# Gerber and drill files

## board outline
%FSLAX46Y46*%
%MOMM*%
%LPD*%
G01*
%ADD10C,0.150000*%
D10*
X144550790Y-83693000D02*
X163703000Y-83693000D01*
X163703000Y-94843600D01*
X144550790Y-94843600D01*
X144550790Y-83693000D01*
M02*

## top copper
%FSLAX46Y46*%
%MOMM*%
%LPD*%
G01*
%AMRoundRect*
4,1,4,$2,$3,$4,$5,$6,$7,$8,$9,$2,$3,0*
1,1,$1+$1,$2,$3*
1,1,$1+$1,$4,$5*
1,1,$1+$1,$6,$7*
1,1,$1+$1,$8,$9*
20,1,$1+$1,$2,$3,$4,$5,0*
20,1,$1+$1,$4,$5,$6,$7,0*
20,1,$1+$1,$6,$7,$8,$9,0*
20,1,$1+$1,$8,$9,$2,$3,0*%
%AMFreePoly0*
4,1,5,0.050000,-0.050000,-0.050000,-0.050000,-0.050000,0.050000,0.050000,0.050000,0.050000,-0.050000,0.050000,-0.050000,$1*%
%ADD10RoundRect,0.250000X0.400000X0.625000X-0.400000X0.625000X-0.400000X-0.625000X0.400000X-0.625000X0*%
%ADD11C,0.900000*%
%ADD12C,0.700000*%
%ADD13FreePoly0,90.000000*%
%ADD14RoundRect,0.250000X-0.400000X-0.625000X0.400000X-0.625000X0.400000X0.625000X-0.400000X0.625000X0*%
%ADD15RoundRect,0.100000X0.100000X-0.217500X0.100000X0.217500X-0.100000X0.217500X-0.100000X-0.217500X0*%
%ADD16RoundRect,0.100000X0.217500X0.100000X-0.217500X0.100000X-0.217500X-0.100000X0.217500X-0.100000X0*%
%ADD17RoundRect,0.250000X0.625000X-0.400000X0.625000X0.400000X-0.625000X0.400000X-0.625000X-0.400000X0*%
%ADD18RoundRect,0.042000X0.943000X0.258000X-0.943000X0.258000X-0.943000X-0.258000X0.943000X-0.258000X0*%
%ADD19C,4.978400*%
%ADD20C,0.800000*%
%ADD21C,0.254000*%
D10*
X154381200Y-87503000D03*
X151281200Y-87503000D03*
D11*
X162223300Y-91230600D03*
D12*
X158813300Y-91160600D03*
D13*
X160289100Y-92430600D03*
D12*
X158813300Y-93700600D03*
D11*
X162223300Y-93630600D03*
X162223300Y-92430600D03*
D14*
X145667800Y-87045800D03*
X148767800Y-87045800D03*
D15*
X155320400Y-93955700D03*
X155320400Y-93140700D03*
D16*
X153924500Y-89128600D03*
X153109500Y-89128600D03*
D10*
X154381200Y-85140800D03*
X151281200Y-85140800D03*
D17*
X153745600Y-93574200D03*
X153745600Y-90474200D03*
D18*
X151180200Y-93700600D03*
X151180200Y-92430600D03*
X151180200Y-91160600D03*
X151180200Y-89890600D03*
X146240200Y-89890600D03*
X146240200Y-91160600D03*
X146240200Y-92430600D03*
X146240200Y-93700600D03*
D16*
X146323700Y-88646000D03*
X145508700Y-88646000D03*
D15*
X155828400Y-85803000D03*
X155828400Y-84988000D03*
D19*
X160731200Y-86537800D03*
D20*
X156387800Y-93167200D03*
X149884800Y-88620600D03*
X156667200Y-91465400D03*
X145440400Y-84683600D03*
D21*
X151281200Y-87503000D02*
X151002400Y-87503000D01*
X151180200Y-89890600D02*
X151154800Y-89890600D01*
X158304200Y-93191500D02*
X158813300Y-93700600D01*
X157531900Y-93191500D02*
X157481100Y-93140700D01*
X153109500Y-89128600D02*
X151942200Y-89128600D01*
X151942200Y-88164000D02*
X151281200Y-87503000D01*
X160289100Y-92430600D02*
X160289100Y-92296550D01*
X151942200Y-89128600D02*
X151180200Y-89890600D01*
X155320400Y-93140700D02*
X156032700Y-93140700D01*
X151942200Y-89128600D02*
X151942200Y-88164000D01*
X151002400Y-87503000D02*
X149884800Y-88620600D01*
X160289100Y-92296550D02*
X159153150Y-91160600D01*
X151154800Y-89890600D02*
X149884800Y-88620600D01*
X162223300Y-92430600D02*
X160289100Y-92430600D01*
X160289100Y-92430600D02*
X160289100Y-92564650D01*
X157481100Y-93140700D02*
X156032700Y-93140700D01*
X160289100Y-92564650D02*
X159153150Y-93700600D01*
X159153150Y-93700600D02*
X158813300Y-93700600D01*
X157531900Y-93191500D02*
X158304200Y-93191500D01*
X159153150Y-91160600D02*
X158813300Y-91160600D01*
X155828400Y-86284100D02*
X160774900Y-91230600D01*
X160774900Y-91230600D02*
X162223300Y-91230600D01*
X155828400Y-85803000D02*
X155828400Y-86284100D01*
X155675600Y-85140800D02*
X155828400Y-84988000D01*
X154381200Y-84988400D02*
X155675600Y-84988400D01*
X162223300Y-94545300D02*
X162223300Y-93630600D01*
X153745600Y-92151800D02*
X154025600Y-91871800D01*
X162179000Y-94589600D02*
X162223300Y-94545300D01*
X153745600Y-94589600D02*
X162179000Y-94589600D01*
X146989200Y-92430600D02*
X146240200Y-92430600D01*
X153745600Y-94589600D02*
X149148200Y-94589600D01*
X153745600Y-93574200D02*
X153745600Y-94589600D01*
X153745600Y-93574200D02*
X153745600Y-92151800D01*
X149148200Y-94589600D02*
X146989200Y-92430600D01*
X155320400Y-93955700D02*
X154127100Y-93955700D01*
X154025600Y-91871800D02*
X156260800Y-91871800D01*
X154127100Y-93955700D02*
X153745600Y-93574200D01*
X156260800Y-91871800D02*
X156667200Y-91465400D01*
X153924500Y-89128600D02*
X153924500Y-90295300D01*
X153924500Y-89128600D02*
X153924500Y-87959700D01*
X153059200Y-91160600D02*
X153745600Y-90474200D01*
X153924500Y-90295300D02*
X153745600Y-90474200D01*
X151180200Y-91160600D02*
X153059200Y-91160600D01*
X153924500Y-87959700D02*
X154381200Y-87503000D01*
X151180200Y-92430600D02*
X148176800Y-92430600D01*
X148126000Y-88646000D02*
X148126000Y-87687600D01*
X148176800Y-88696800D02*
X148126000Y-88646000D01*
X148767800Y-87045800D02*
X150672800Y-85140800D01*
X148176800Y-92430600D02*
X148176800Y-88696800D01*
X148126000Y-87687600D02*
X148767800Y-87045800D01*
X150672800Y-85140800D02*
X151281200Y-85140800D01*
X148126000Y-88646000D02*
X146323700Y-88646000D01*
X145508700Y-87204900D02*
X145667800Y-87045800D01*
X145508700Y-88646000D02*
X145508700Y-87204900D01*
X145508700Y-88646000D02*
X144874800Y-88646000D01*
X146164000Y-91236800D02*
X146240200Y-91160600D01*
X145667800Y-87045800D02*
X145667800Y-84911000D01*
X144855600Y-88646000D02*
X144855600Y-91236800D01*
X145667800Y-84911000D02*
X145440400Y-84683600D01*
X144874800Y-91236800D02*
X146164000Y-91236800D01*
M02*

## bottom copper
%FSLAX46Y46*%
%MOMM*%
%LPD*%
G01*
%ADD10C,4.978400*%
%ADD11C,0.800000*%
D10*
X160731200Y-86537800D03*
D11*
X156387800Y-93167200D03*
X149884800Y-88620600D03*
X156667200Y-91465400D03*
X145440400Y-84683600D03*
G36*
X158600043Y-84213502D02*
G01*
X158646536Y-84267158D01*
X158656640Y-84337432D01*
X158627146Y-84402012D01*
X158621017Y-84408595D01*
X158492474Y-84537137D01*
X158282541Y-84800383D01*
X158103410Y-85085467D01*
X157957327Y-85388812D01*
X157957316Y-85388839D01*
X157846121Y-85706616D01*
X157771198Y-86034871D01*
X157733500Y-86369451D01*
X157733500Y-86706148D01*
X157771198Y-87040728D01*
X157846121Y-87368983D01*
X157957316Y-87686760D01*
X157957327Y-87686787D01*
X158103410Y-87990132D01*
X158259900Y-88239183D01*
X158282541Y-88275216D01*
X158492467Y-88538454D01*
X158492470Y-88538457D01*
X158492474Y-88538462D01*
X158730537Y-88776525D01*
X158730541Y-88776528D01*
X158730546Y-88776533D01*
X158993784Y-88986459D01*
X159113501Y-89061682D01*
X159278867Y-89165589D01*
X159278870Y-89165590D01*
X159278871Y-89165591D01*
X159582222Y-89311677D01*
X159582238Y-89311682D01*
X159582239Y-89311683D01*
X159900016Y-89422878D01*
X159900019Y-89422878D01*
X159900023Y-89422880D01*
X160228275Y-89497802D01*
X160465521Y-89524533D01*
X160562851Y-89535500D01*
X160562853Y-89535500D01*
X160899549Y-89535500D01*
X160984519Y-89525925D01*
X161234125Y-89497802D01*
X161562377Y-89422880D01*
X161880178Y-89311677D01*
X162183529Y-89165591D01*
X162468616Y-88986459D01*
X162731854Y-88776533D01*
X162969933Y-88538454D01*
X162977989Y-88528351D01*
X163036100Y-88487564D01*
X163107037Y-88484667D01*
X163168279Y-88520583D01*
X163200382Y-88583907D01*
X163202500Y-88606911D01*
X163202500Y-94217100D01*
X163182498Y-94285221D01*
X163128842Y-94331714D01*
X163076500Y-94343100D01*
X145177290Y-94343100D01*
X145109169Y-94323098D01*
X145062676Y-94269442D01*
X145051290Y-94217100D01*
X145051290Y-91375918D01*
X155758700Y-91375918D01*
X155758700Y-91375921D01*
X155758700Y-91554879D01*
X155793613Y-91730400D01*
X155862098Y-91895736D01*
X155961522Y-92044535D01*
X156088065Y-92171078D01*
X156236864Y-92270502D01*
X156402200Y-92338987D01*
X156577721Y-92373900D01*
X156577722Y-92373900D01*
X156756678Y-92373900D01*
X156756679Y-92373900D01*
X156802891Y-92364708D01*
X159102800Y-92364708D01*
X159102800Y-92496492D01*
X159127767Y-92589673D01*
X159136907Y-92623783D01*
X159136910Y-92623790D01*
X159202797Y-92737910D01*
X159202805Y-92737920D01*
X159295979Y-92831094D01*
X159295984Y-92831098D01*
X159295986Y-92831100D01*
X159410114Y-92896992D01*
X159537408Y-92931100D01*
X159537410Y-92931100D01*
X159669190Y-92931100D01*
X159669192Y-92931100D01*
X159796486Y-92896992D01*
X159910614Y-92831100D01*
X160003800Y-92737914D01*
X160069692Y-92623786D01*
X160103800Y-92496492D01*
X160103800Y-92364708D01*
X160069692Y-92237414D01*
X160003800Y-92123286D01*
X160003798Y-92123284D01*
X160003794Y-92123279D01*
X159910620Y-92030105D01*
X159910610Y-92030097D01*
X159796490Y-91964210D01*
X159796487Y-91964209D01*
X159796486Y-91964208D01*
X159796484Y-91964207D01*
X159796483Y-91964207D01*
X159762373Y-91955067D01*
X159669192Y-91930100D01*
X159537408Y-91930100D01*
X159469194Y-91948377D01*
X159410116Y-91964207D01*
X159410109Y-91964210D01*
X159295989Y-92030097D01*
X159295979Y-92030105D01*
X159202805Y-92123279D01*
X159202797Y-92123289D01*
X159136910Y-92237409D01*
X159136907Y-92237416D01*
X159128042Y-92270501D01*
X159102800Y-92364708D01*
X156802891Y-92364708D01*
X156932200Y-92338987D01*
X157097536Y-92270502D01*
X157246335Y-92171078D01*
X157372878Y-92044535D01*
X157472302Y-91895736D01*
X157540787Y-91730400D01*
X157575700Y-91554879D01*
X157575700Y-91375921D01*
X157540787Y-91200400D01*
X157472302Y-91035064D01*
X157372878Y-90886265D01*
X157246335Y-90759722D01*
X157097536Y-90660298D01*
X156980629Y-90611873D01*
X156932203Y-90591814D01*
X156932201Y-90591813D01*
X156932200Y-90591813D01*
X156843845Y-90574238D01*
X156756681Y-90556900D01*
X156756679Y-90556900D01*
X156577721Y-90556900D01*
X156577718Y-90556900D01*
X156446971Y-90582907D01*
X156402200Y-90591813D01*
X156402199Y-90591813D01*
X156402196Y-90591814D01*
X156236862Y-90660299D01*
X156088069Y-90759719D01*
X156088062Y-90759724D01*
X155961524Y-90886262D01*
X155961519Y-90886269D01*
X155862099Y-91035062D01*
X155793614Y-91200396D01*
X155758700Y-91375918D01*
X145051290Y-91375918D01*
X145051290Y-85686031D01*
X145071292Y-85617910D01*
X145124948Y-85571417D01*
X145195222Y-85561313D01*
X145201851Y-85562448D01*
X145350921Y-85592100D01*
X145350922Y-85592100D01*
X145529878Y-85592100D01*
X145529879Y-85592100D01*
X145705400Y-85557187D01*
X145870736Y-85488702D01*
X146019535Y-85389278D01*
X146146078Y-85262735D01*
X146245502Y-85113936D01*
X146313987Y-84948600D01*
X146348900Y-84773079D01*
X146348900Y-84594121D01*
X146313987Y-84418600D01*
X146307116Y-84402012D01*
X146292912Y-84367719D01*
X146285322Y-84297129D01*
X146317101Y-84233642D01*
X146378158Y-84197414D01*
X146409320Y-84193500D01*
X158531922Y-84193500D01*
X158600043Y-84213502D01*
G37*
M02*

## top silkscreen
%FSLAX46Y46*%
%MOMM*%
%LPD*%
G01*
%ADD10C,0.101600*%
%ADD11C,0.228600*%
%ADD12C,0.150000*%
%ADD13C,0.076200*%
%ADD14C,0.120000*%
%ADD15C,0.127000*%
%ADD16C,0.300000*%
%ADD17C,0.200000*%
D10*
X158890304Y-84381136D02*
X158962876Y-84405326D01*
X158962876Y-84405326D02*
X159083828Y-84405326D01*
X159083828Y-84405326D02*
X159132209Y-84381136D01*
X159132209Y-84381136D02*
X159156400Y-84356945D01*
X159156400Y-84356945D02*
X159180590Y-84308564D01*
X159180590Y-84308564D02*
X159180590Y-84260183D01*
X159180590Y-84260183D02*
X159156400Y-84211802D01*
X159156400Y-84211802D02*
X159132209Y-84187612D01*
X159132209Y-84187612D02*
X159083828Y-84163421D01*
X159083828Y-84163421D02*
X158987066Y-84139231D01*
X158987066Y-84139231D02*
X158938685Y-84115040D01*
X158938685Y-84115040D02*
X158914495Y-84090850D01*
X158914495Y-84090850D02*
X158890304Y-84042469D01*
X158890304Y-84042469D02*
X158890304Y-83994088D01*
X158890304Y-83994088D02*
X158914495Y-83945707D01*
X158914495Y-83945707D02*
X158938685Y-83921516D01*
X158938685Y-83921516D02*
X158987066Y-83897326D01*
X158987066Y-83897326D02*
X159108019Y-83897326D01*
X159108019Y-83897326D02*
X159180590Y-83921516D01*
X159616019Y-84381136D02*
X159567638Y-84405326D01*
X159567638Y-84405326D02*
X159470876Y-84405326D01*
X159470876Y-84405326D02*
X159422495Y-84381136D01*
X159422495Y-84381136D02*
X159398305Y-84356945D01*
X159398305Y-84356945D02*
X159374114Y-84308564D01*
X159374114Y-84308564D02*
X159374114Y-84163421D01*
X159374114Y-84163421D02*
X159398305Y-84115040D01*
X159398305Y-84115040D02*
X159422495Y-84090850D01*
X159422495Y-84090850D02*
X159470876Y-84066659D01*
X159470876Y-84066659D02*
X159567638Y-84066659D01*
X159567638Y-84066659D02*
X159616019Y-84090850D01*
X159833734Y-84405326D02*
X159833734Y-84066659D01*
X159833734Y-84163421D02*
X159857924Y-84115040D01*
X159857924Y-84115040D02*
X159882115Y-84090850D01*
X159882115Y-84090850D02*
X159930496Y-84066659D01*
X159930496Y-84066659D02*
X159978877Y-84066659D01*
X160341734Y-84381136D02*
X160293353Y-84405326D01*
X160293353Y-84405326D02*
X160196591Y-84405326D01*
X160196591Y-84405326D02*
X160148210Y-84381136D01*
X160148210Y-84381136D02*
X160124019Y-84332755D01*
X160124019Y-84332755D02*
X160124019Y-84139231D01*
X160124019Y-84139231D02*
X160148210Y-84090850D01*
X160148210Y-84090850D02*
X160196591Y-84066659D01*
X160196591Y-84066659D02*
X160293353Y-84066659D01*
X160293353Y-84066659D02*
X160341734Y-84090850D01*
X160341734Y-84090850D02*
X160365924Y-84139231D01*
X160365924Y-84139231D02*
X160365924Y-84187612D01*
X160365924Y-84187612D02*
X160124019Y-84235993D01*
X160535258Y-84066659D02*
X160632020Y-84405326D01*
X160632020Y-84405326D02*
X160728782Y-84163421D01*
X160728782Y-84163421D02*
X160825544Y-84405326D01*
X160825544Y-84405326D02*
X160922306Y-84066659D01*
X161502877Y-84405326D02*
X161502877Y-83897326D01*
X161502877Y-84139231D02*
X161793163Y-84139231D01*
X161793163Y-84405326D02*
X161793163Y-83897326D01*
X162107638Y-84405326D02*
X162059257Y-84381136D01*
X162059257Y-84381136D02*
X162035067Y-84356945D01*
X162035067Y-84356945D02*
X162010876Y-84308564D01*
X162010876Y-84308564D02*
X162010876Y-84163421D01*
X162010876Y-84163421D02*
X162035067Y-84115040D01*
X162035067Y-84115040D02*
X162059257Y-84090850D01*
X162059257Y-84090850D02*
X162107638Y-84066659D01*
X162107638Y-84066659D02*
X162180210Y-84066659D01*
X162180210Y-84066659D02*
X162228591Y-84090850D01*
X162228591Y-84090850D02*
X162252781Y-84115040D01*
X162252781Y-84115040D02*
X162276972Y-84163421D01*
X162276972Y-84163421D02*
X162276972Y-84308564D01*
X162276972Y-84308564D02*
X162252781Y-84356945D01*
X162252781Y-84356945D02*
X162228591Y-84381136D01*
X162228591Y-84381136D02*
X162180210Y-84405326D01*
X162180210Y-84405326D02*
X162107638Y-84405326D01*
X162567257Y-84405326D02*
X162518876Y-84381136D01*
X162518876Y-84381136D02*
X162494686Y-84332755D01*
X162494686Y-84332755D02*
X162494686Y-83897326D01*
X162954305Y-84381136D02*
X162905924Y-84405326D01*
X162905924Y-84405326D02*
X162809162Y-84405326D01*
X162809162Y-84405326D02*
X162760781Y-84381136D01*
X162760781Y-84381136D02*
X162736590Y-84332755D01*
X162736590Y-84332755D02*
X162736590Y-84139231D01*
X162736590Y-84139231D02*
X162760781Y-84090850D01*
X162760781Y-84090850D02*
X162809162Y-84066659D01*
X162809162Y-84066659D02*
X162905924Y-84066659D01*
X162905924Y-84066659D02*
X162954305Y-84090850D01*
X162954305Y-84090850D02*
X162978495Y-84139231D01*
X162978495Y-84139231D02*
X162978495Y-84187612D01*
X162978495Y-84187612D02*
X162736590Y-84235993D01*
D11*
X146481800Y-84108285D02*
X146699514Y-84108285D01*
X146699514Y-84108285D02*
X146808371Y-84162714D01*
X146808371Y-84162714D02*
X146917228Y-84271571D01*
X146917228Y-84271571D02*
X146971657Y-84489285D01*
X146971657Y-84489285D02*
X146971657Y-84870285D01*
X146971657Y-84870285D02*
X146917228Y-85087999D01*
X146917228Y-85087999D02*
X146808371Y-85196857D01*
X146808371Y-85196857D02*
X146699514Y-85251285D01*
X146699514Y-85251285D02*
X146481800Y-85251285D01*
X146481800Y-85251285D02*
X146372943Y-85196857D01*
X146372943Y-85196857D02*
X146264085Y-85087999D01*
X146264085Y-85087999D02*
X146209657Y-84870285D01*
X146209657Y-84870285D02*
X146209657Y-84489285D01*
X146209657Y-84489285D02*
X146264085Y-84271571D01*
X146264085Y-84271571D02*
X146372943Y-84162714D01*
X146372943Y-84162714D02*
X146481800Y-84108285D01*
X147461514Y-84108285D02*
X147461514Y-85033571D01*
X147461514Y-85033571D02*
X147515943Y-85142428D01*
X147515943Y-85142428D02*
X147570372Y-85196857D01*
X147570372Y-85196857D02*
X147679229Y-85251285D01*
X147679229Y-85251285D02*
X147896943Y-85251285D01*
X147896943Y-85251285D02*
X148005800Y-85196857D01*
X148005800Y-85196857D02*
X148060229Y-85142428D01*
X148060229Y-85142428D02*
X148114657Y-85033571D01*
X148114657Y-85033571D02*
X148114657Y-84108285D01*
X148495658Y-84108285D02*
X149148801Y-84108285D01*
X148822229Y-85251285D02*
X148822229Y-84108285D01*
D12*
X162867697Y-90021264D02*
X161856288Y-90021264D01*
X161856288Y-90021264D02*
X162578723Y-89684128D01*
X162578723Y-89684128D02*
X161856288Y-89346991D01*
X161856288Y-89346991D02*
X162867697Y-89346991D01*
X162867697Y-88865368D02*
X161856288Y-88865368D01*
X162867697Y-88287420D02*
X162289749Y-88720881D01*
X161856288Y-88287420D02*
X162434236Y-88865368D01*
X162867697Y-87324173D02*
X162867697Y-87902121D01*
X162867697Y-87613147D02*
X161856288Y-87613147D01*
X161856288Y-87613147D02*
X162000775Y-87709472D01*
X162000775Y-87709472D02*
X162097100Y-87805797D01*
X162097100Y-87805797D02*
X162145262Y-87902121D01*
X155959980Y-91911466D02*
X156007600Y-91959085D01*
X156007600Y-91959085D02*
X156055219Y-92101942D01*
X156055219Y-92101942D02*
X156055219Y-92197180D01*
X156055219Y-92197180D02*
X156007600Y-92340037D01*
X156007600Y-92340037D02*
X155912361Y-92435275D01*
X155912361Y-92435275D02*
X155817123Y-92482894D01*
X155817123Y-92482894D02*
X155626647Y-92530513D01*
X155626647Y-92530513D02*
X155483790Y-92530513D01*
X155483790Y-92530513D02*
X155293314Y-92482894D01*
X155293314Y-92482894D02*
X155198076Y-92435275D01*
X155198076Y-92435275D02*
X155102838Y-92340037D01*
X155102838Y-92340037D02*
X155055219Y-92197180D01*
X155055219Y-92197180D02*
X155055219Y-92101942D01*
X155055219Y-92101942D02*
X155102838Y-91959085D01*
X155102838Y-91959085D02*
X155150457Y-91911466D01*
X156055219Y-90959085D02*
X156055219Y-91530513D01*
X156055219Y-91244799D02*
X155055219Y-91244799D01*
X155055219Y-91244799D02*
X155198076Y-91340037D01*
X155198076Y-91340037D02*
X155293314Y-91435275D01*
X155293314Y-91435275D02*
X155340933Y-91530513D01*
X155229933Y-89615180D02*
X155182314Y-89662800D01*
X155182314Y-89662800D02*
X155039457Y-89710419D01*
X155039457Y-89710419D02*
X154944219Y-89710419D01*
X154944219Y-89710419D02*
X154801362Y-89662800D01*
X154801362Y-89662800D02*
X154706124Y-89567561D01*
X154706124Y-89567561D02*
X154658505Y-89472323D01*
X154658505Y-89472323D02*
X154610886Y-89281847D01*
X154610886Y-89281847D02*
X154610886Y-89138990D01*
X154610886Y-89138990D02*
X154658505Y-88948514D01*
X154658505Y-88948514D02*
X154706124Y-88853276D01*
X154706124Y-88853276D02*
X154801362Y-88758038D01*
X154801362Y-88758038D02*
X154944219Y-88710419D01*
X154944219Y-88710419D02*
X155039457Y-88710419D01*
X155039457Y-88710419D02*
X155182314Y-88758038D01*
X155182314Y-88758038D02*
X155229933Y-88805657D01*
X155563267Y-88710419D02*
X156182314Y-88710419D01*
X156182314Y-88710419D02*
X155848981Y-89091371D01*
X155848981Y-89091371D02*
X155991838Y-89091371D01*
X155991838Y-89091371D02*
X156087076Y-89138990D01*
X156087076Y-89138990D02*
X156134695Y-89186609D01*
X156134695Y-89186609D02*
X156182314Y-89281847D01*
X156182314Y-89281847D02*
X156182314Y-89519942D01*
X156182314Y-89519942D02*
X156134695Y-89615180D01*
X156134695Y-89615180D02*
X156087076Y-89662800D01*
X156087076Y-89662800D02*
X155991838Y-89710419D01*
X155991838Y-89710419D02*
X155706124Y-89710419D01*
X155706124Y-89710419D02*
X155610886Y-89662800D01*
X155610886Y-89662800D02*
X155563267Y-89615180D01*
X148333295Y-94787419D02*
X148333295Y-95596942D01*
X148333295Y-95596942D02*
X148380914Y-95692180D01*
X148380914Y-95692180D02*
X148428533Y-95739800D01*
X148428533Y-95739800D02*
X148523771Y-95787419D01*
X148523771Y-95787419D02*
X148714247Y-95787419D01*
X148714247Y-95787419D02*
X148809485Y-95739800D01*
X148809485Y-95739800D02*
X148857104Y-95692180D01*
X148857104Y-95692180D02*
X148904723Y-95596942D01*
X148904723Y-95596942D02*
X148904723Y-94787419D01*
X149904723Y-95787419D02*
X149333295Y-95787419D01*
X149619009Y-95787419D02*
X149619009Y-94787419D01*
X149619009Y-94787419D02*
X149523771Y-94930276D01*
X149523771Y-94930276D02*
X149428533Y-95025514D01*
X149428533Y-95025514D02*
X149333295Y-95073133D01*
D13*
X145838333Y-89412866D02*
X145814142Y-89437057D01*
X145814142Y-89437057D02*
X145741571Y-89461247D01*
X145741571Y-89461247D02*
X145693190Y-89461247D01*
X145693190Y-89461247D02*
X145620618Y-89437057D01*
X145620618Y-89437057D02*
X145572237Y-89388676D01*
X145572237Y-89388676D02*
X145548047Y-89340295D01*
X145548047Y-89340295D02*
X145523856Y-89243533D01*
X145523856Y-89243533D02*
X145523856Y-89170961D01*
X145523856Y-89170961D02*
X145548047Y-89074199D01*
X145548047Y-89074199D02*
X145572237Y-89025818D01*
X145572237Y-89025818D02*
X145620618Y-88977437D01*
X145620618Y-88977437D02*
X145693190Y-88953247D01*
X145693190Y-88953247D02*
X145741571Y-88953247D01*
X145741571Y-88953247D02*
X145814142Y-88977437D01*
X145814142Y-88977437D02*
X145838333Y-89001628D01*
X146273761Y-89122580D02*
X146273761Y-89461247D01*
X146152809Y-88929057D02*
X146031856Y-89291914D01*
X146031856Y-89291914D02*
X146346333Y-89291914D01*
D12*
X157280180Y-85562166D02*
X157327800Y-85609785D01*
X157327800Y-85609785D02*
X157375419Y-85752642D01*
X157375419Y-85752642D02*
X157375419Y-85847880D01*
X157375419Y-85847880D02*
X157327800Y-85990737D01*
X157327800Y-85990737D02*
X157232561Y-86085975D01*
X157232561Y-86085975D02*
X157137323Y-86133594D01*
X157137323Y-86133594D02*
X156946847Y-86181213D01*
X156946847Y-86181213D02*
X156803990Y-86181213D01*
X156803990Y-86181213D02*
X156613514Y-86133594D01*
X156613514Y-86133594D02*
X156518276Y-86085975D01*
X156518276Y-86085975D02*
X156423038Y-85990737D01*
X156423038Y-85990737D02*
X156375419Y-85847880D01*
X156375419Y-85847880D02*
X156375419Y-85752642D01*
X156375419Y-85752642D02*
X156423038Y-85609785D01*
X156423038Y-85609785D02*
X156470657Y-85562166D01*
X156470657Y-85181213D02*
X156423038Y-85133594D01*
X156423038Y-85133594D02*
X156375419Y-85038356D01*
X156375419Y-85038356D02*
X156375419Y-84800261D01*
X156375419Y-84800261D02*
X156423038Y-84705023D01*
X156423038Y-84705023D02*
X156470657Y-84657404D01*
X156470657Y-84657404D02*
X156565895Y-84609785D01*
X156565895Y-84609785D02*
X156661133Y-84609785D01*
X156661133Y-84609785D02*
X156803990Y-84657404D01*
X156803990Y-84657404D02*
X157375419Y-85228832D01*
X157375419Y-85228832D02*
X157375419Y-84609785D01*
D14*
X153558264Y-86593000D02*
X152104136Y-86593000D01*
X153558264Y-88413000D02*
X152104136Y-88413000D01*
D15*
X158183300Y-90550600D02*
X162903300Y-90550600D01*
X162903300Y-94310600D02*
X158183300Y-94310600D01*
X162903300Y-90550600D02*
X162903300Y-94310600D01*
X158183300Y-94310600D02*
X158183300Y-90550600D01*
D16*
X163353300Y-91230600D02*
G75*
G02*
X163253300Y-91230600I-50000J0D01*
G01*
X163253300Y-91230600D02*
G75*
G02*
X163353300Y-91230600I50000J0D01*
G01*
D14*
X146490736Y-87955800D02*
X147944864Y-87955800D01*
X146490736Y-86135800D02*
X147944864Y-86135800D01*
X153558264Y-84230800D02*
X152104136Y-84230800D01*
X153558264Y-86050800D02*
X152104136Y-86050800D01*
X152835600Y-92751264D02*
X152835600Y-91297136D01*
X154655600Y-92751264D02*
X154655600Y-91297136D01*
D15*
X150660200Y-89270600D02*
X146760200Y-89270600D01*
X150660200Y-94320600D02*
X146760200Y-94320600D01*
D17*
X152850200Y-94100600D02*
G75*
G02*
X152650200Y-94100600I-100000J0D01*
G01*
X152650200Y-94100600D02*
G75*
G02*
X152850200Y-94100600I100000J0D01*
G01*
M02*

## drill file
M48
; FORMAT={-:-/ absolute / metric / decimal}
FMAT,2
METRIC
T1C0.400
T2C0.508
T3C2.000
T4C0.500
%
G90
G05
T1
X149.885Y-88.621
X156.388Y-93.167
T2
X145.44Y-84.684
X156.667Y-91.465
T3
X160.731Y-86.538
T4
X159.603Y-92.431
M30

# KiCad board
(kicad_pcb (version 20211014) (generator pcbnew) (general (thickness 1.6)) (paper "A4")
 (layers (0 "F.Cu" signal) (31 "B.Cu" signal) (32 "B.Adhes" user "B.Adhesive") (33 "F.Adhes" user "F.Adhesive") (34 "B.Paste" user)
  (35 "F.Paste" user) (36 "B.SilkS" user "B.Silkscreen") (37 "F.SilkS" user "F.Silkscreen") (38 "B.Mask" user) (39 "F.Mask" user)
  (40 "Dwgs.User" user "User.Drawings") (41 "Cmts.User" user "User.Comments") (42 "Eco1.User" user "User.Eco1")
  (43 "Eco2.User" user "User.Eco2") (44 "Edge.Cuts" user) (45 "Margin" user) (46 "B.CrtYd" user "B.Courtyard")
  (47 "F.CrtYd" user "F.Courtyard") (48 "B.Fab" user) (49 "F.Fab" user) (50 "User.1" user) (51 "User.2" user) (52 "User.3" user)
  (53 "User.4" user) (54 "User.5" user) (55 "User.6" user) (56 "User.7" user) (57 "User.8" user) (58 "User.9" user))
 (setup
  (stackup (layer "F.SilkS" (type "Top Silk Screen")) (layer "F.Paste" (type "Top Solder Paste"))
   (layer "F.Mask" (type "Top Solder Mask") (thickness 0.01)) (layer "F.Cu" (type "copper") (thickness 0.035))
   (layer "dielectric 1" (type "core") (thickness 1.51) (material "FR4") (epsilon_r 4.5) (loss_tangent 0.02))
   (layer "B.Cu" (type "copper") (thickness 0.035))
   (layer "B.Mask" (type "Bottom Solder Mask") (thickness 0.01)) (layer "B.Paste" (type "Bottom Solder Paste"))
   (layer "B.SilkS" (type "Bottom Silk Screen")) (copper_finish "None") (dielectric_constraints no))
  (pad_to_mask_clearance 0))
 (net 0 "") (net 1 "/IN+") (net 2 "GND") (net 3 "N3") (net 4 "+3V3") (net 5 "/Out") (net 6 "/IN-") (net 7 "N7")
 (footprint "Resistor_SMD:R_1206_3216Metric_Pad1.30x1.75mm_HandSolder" (layer "F.Cu") (at 152.8312 87.503 180)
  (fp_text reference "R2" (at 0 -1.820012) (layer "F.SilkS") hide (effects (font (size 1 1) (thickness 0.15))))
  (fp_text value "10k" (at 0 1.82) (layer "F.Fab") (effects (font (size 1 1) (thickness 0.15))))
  (fp_line (start -0.727064 0.91) (end 0.727064 0.91) (layer "F.SilkS") (width 0.12))
  (fp_line (start -0.727064 -0.91) (end 0.727064 -0.91) (layer "F.SilkS") (width 0.12))
  (pad "1" smd roundrect (at -1.55 0 180) (size 1.3 1.75) (layers "F.Cu" "F.Paste" "F.Mask") (roundrect_rratio 0.1923076923) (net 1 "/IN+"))
  (pad "2" smd roundrect (at 1.55 0 180) (size 1.3 1.75) (layers "F.Cu" "F.Paste" "F.Mask") (roundrect_rratio 0.1923076923) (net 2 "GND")))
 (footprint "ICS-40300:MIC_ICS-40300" (layer "F.Cu") (at 159.6033 92.4306 -90)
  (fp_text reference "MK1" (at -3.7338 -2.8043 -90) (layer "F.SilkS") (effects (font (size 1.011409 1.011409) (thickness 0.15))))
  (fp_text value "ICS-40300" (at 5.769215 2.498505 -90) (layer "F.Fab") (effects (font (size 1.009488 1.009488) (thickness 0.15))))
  (fp_line (start -1.88 1.42) (end -1.88 -3.3) (layer "F.SilkS") (width 0.127))
  (fp_line (start 1.88 -3.3) (end 1.88 1.42) (layer "F.SilkS") (width 0.127))
  (fp_line (start -1.88 -3.3) (end 1.88 -3.3) (layer "F.SilkS") (width 0.127))
  (fp_line (start 1.88 1.42) (end -1.88 1.42) (layer "F.SilkS") (width 0.127))
  (fp_circle (center -1.2 -3.7) (end -1.15 -3.7) (layer "F.SilkS") (width 0.3) (fill none))
  (pad "" np_thru_hole circle (at 0 0 270) (size 0.5 0.5) (drill 0.5) (layers *.Cu *.Mask))
  (pad "1" smd circle (at -1.2 -2.62 180) (size 0.9 0.9) (layers "F.Cu" "F.Mask") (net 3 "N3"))
  (pad "2" smd circle (at -1.27 0.79 180) (size 0.7 0.7) (layers "F.Cu" "F.Mask") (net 2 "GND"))
  (pad "3" smd custom (at 0 -0.6858 90) (size 0.1 0.1) (layers "F.Cu") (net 2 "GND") (zone_connect 0)
   (options (clearance outline) (anchor rect)) (primitives))
  (pad "4" smd circle (at 1.27 0.79 180) (size 0.7 0.7) (layers "F.Cu" "F.Mask") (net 2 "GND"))
  (pad "5" smd circle (at 1.2 -2.62 180) (size 0.9 0.9) (layers "F.Cu" "F.Mask") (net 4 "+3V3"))
  (pad "6" smd circle (at 0 -2.62 180) (size 0.9 0.9) (layers "F.Cu" "F.Mask") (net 2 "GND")))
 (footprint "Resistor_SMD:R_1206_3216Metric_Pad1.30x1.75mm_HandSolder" (layer "F.Cu") (at 147.2178 87.0458)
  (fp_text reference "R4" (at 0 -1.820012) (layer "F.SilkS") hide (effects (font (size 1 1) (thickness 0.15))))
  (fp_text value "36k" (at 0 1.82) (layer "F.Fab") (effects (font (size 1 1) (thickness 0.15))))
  (fp_line (start -0.727064 0.91) (end 0.727064 0.91) (layer "F.SilkS") (width 0.12))
  (fp_line (start -0.727064 -0.91) (end 0.727064 -0.91) (layer "F.SilkS") (width 0.12))
  (pad "1" smd roundrect (at -1.55 0) (size 1.3 1.75) (layers "F.Cu" "F.Paste" "F.Mask") (roundrect_rratio 0.1923076923) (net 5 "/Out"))
  (pad "2" smd roundrect (at 1.55 0) (size 1.3 1.75) (layers "F.Cu" "F.Paste" "F.Mask") (roundrect_rratio 0.1923076923) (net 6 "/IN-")))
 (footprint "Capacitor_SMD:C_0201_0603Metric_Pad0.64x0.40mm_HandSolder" (layer "F.Cu") (at 155.3204 93.5482 90)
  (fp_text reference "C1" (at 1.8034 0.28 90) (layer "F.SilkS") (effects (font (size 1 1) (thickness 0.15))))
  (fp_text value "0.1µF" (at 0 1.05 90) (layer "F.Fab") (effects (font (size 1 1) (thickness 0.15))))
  (pad "" smd roundrect (at 0.4325 0 90) (size 0.458 0.36) (layers "F.Paste") (roundrect_rratio 0.25))
  (pad "" smd roundrect (at -0.4325 0 90) (size 0.458 0.36) (layers "F.Paste") (roundrect_rratio 0.25))
  (pad "1" smd roundrect (at -0.4075 0 90) (size 0.635 0.4) (layers "F.Cu" "F.Mask") (roundrect_rratio 0.25) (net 4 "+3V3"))
  (pad "2" smd roundrect (at 0.4075 0 90) (size 0.635 0.4) (layers "F.Cu" "F.Mask") (roundrect_rratio 0.25) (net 2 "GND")))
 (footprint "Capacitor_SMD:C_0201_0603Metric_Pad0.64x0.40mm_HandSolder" (layer "F.Cu") (at 153.517 89.1286 180)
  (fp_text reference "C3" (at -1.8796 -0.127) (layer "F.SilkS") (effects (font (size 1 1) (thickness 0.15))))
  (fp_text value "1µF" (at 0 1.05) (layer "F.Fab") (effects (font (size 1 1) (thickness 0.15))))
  (pad "" smd roundrect (at -0.4325 0 180) (size 0.458 0.36) (layers "F.Paste") (roundrect_rratio 0.25))
  (pad "" smd roundrect (at 0.4325 0 180) (size 0.458 0.36) (layers "F.Paste") (roundrect_rratio 0.25))
  (pad "1" smd roundrect (at -0.4075 0 180) (size 0.635 0.4) (layers "F.Cu" "F.Mask") (roundrect_rratio 0.25) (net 1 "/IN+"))
  (pad "2" smd roundrect (at 0.4075 0 180) (size 0.635 0.4) (layers "F.Cu" "F.Mask") (roundrect_rratio 0.25) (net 2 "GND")))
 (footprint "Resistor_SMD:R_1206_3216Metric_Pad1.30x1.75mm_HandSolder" (layer "F.Cu") (at 152.8312 85.1408 180)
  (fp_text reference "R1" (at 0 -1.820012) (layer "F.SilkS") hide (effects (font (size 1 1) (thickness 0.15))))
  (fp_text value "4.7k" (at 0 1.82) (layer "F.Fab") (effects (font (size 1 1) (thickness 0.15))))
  (fp_line (start -0.727064 0.91) (end 0.727064 0.91) (layer "F.SilkS") (width 0.12))
  (fp_line (start -0.727064 -0.91) (end 0.727064 -0.91) (layer "F.SilkS") (width 0.12))
  (pad "1" smd roundrect (at -1.55 0 180) (size 1.3 1.75) (layers "F.Cu" "F.Paste" "F.Mask") (roundrect_rratio 0.1923076923) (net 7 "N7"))
  (pad "2" smd roundrect (at 1.55 0 180) (size 1.3 1.75) (layers "F.Cu" "F.Paste" "F.Mask") (roundrect_rratio 0.1923076923) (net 6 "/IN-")))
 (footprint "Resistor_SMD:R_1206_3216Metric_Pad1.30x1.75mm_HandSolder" (layer "F.Cu") (at 153.7456 92.0242 90)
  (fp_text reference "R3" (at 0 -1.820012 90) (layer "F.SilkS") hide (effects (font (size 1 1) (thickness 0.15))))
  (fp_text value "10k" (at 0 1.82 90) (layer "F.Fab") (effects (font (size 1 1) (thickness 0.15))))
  (fp_line (start -0.727064 -0.91) (end 0.727064 -0.91) (layer "F.SilkS") (width 0.12))
  (fp_line (start -0.727064 0.91) (end 0.727064 0.91) (layer "F.SilkS") (width 0.12))
  (pad "1" smd roundrect (at -1.55 0 90) (size 1.3 1.75) (layers "F.Cu" "F.Paste" "F.Mask") (roundrect_rratio 0.1923076923) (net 4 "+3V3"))
  (pad "2" smd roundrect (at 1.55 0 90) (size 1.3 1.75) (layers "F.Cu" "F.Paste" "F.Mask") (roundrect_rratio 0.1923076923) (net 1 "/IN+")))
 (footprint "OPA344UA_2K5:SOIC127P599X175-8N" (layer "F.Cu") (at 148.7102 91.7956 180)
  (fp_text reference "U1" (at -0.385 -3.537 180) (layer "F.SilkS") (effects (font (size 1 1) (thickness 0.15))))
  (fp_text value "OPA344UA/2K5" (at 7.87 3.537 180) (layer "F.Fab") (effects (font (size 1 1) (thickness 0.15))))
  (fp_line (start -1.95 2.525) (end 1.95 2.525) (layer "F.SilkS") (width 0.127))
  (fp_line (start -1.95 -2.525) (end 1.95 -2.525) (layer "F.SilkS") (width 0.127))
  (fp_circle (center -4.04 -2.305) (end -3.94 -2.305) (layer "F.SilkS") (width 0.2) (fill none))
  (pad "1" smd roundrect locked (at -2.47 -1.905 180) (size 1.97 0.6) (layers "F.Cu" "F.Paste" "F.Mask") (roundrect_rratio 0.07))
  (pad "2" smd roundrect locked (at -2.47 -0.635 180) (size 1.97 0.6) (layers "F.Cu" "F.Paste" "F.Mask") (roundrect_rratio 0.07)
   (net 6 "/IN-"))
  (pad "3" smd roundrect locked (at -2.47 0.635 180) (size 1.97 0.6) (layers "F.Cu" "F.Paste" "F.Mask") (roundrect_rratio 0.07)
   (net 1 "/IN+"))
  (pad "4" smd roundrect locked (at -2.47 1.905 180) (size 1.97 0.6) (layers "F.Cu" "F.Paste" "F.Mask") (roundrect_rratio 0.07)
   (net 2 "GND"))
  (pad "5" smd roundrect locked (at 2.47 1.905 180) (size 1.97 0.6) (layers "F.Cu" "F.Paste" "F.Mask") (roundrect_rratio 0.07))
  (pad "6" smd roundrect locked (at 2.47 0.635 180) (size 1.97 0.6) (layers "F.Cu" "F.Paste" "F.Mask") (roundrect_rratio 0.07)
   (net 5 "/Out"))
  (pad "7" smd roundrect locked (at 2.47 -0.635 180) (size 1.97 0.6) (layers "F.Cu" "F.Paste" "F.Mask") (roundrect_rratio 0.07)
   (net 4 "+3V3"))
  (pad "8" smd roundrect locked (at 2.47 -1.905 180) (size 1.97 0.6) (layers "F.Cu" "F.Paste" "F.Mask") (roundrect_rratio 0.07)))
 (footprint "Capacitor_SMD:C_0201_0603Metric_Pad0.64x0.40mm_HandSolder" (layer "F.Cu") (at 145.9162 88.646 180)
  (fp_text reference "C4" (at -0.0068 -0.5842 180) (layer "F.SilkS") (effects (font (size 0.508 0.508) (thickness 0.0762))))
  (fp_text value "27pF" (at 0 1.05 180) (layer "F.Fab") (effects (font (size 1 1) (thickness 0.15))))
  (pad "" smd roundrect (at -0.4325 0 180) (size 0.458 0.36) (layers "F.Paste") (roundrect_rratio 0.25))
  (pad "" smd roundrect (at 0.4325 0 180) (size 0.458 0.36) (layers "F.Paste") (roundrect_rratio 0.25))
  (pad "1" smd roundrect (at -0.4075 0 180) (size 0.635 0.4) (layers "F.Cu" "F.Mask") (roundrect_rratio 0.25) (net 6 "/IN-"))
  (pad "2" smd roundrect (at 0.4075 0 180) (size 0.635 0.4) (layers "F.Cu" "F.Mask") (roundrect_rratio 0.25) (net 5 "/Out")))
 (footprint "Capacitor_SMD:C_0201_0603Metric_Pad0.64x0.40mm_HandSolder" (layer "F.Cu") (at 155.8284 85.3955 90)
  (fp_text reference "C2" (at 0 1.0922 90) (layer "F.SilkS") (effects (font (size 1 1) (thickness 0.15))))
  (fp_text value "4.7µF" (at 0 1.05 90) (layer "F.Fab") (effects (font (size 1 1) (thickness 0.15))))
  (pad "" smd roundrect (at -0.4325 0 90) (size 0.458 0.36) (layers "F.Paste") (roundrect_rratio 0.25))
  (pad "" smd roundrect (at 0.4325 0 90) (size 0.458 0.36) (layers "F.Paste") (roundrect_rratio 0.25))
  (pad "1" smd roundrect (at -0.4075 0 90) (size 0.635 0.4) (layers "F.Cu" "F.Mask") (roundrect_rratio 0.25) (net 3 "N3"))
  (pad "2" smd roundrect (at 0.4075 0 90) (size 0.635 0.4) (layers "F.Cu" "F.Mask") (roundrect_rratio 0.25) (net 7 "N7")))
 (gr_rect (start 144.55079 94.8436) (end 163.703 83.693) (layer "Edge.Cuts") (width 0.15) (fill none))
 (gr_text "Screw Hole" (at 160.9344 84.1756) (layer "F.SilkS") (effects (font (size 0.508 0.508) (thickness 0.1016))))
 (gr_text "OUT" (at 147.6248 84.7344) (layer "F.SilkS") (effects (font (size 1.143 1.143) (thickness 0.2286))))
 (via (at 160.7312 86.5378) (size 4.9784) (drill 2.000001) (layers "F.Cu" "B.Cu") (free) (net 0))
 (segment (start 151.2812 87.503) (end 151.0024 87.503) (width 0.254) (layer "F.Cu") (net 2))
 (segment (start 151.1802 89.8906) (end 151.1548 89.8906) (width 0.254) (layer "F.Cu") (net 2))
 (segment (start 158.3042 93.1915) (end 158.8133 93.7006) (width 0.254) (layer "F.Cu") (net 2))
 (segment (start 157.5319 93.1915) (end 157.4811 93.1407) (width 0.254) (layer "F.Cu") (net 2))
 (segment (start 153.1095 89.1286) (end 151.9422 89.1286) (width 0.254) (layer "F.Cu") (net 2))
 (segment (start 151.9422 88.164) (end 151.2812 87.503) (width 0.254) (layer "F.Cu") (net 2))
 (segment (start 160.2891 92.4306) (end 160.2891 92.29655) (width 0.254) (layer "F.Cu") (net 2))
 (segment (start 151.9422 89.1286) (end 151.1802 89.8906) (width 0.254) (layer "F.Cu") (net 2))
 (segment (start 155.3204 93.1407) (end 156.0327 93.1407) (width 0.254) (layer "F.Cu") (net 2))
 (segment (start 151.9422 89.1286) (end 151.9422 88.164) (width 0.254) (layer "F.Cu") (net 2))
 (segment (start 151.0024 87.503) (end 149.8848 88.6206) (width 0.254) (layer "F.Cu") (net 2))
 (segment (start 160.2891 92.29655) (end 159.15315 91.1606) (width 0.254) (layer "F.Cu") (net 2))
 (segment (start 151.1548 89.8906) (end 149.8848 88.6206) (width 0.254) (layer "F.Cu") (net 2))
 (segment (start 162.2233 92.4306) (end 160.2891 92.4306) (width 0.254) (layer "F.Cu") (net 2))
 (segment (start 160.2891 92.4306) (end 160.2891 92.56465) (width 0.254) (layer "F.Cu") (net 2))
 (segment (start 157.4811 93.1407) (end 156.0327 93.1407) (width 0.254) (layer "F.Cu") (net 2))
 (segment (start 160.2891 92.56465) (end 159.15315 93.7006) (width 0.254) (layer "F.Cu") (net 2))
 (segment (start 159.15315 93.7006) (end 158.8133 93.7006) (width 0.254) (layer "F.Cu") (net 2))
 (segment (start 157.5319 93.1915) (end 158.3042 93.1915) (width 0.254) (layer "F.Cu") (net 2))
 (segment (start 159.15315 91.1606) (end 158.8133 91.1606) (width 0.254) (layer "F.Cu") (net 2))
 (via (at 156.3878 93.1672) (size 0.8) (drill 0.4) (layers "F.Cu" "B.Cu") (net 2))
 (via (at 149.8848 88.6206) (size 0.8) (drill 0.4) (layers "F.Cu" "B.Cu") (free) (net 2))
 (segment (start 155.8284 86.2841) (end 160.7749 91.2306) (width 0.254) (layer "F.Cu") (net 3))
 (segment (start 160.7749 91.2306) (end 162.2233 91.2306) (width 0.254) (layer "F.Cu") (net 3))
 (segment (start 155.8284 85.803) (end 155.8284 86.2841) (width 0.254) (layer "F.Cu") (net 3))
 (segment (start 155.6756 85.1408) (end 155.8284 84.988) (width 0.254) (layer "F.Cu") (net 7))
 (segment (start 154.3812 84.9884) (end 155.6756 84.9884) (width 0.254) (layer "F.Cu") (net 7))
 (segment (start 162.2233 94.5453) (end 162.2233 93.6306) (width 0.254) (layer "F.Cu") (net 4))
 (segment (start 153.7456 92.1518) (end 154.0256 91.8718) (width 0.254) (layer "F.Cu") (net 4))
 (segment (start 162.179 94.5896) (end 162.2233 94.5453) (width 0.254) (layer "F.Cu") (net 4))
 (segment (start 153.7456 94.5896) (end 162.179 94.5896) (width 0.254) (layer "F.Cu") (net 4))
 (segment (start 146.9892 92.4306) (end 146.2402 92.4306) (width 0.254) (layer "F.Cu") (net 4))
 (segment (start 153.7456 94.5896) (end 149.1482 94.5896) (width 0.254) (layer "F.Cu") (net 4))
 (segment (start 153.7456 93.5742) (end 153.7456 94.5896) (width 0.254) (layer "F.Cu") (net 4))
 (segment (start 153.7456 93.5742) (end 153.7456 92.1518) (width 0.254) (layer "F.Cu") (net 4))
 (segment (start 149.1482 94.5896) (end 146.9892 92.4306) (width 0.254) (layer "F.Cu") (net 4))
 (segment (start 155.3204 93.9557) (end 154.1271 93.9557) (width 0.254) (layer "F.Cu") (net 4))
 (segment (start 154.0256 91.8718) (end 156.2608 91.8718) (width 0.254) (layer "F.Cu") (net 4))
 (segment (start 154.1271 93.9557) (end 153.7456 93.5742) (width 0.254) (layer "F.Cu") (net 4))
 (segment (start 156.2608 91.8718) (end 156.6672 91.4654) (width 0.254) (layer "F.Cu") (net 4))
 (via (at 156.6672 91.4654) (size 0.8) (drill 0.508) (layers "F.Cu" "B.Cu") (free) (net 4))
 (segment (start 153.9245 89.1286) (end 153.9245 90.2953) (width 0.254) (layer "F.Cu") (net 1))
 (segment (start 153.9245 89.1286) (end 153.9245 87.9597) (width 0.254) (layer "F.Cu") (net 1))
 (segment (start 153.0592 91.1606) (end 153.7456 90.4742) (width 0.254) (layer "F.Cu") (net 1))
 (segment (start 153.9245 90.2953) (end 153.7456 90.4742) (width 0.254) (layer "F.Cu") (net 1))
 (segment (start 151.1802 91.1606) (end 153.0592 91.1606) (width 0.254) (layer "F.Cu") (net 1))
 (segment (start 153.9245 87.9597) (end 154.3812 87.503) (width 0.254) (layer "F.Cu") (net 1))
 (segment (start 151.1802 92.4306) (end 148.1768 92.4306) (width 0.254) (layer "F.Cu") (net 6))
 (segment (start 148.126 88.646) (end 148.126 87.6876) (width 0.254) (layer "F.Cu") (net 6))
 (segment (start 148.1768 88.6968) (end 148.126 88.646) (width 0.254) (layer "F.Cu") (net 6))
 (segment (start 148.7678 87.0458) (end 150.6728 85.1408) (width 0.254) (layer "F.Cu") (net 6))
 (segment (start 148.1768 92.4306) (end 148.1768 88.6968) (width 0.254) (layer "F.Cu") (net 6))
 (segment (start 148.126 87.6876) (end 148.7678 87.0458) (width 0.254) (layer "F.Cu") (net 6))
 (segment (start 150.6728 85.1408) (end 151.2812 85.1408) (width 0.254) (layer "F.Cu") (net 6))
 (segment (start 148.126 88.646) (end 146.3237 88.646) (width 0.254) (layer "F.Cu") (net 6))
 (segment (start 145.5087 87.2049) (end 145.6678 87.0458) (width 0.254) (layer "F.Cu") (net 5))
 (segment (start 145.5087 88.646) (end 145.5087 87.2049) (width 0.254) (layer "F.Cu") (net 5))
 (segment (start 145.5087 88.646) (end 144.8748 88.646) (width 0.254) (layer "F.Cu") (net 5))
 (segment (start 146.164 91.2368) (end 146.2402 91.1606) (width 0.254) (layer "F.Cu") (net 5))
 (segment (start 145.6678 87.0458) (end 145.6678 84.911) (width 0.254) (layer "F.Cu") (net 5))
 (segment (start 144.8556 88.646) (end 144.8556 91.2368) (width 0.254) (layer "F.Cu") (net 5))
 (segment (start 145.6678 84.911) (end 145.4404 84.6836) (width 0.254) (layer "F.Cu") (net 5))
 (segment (start 144.8748 91.2368) (end 146.164 91.2368) (width 0.254) (layer "F.Cu") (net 5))
 (via (at 145.4404 84.6836) (size 0.8) (drill 0.508) (layers "F.Cu" "B.Cu") (free) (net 5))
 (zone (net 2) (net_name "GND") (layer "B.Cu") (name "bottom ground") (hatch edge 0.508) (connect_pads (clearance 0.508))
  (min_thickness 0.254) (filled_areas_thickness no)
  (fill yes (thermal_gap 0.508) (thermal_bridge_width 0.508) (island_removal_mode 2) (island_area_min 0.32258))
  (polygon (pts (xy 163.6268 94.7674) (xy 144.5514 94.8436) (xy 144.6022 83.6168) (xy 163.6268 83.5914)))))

